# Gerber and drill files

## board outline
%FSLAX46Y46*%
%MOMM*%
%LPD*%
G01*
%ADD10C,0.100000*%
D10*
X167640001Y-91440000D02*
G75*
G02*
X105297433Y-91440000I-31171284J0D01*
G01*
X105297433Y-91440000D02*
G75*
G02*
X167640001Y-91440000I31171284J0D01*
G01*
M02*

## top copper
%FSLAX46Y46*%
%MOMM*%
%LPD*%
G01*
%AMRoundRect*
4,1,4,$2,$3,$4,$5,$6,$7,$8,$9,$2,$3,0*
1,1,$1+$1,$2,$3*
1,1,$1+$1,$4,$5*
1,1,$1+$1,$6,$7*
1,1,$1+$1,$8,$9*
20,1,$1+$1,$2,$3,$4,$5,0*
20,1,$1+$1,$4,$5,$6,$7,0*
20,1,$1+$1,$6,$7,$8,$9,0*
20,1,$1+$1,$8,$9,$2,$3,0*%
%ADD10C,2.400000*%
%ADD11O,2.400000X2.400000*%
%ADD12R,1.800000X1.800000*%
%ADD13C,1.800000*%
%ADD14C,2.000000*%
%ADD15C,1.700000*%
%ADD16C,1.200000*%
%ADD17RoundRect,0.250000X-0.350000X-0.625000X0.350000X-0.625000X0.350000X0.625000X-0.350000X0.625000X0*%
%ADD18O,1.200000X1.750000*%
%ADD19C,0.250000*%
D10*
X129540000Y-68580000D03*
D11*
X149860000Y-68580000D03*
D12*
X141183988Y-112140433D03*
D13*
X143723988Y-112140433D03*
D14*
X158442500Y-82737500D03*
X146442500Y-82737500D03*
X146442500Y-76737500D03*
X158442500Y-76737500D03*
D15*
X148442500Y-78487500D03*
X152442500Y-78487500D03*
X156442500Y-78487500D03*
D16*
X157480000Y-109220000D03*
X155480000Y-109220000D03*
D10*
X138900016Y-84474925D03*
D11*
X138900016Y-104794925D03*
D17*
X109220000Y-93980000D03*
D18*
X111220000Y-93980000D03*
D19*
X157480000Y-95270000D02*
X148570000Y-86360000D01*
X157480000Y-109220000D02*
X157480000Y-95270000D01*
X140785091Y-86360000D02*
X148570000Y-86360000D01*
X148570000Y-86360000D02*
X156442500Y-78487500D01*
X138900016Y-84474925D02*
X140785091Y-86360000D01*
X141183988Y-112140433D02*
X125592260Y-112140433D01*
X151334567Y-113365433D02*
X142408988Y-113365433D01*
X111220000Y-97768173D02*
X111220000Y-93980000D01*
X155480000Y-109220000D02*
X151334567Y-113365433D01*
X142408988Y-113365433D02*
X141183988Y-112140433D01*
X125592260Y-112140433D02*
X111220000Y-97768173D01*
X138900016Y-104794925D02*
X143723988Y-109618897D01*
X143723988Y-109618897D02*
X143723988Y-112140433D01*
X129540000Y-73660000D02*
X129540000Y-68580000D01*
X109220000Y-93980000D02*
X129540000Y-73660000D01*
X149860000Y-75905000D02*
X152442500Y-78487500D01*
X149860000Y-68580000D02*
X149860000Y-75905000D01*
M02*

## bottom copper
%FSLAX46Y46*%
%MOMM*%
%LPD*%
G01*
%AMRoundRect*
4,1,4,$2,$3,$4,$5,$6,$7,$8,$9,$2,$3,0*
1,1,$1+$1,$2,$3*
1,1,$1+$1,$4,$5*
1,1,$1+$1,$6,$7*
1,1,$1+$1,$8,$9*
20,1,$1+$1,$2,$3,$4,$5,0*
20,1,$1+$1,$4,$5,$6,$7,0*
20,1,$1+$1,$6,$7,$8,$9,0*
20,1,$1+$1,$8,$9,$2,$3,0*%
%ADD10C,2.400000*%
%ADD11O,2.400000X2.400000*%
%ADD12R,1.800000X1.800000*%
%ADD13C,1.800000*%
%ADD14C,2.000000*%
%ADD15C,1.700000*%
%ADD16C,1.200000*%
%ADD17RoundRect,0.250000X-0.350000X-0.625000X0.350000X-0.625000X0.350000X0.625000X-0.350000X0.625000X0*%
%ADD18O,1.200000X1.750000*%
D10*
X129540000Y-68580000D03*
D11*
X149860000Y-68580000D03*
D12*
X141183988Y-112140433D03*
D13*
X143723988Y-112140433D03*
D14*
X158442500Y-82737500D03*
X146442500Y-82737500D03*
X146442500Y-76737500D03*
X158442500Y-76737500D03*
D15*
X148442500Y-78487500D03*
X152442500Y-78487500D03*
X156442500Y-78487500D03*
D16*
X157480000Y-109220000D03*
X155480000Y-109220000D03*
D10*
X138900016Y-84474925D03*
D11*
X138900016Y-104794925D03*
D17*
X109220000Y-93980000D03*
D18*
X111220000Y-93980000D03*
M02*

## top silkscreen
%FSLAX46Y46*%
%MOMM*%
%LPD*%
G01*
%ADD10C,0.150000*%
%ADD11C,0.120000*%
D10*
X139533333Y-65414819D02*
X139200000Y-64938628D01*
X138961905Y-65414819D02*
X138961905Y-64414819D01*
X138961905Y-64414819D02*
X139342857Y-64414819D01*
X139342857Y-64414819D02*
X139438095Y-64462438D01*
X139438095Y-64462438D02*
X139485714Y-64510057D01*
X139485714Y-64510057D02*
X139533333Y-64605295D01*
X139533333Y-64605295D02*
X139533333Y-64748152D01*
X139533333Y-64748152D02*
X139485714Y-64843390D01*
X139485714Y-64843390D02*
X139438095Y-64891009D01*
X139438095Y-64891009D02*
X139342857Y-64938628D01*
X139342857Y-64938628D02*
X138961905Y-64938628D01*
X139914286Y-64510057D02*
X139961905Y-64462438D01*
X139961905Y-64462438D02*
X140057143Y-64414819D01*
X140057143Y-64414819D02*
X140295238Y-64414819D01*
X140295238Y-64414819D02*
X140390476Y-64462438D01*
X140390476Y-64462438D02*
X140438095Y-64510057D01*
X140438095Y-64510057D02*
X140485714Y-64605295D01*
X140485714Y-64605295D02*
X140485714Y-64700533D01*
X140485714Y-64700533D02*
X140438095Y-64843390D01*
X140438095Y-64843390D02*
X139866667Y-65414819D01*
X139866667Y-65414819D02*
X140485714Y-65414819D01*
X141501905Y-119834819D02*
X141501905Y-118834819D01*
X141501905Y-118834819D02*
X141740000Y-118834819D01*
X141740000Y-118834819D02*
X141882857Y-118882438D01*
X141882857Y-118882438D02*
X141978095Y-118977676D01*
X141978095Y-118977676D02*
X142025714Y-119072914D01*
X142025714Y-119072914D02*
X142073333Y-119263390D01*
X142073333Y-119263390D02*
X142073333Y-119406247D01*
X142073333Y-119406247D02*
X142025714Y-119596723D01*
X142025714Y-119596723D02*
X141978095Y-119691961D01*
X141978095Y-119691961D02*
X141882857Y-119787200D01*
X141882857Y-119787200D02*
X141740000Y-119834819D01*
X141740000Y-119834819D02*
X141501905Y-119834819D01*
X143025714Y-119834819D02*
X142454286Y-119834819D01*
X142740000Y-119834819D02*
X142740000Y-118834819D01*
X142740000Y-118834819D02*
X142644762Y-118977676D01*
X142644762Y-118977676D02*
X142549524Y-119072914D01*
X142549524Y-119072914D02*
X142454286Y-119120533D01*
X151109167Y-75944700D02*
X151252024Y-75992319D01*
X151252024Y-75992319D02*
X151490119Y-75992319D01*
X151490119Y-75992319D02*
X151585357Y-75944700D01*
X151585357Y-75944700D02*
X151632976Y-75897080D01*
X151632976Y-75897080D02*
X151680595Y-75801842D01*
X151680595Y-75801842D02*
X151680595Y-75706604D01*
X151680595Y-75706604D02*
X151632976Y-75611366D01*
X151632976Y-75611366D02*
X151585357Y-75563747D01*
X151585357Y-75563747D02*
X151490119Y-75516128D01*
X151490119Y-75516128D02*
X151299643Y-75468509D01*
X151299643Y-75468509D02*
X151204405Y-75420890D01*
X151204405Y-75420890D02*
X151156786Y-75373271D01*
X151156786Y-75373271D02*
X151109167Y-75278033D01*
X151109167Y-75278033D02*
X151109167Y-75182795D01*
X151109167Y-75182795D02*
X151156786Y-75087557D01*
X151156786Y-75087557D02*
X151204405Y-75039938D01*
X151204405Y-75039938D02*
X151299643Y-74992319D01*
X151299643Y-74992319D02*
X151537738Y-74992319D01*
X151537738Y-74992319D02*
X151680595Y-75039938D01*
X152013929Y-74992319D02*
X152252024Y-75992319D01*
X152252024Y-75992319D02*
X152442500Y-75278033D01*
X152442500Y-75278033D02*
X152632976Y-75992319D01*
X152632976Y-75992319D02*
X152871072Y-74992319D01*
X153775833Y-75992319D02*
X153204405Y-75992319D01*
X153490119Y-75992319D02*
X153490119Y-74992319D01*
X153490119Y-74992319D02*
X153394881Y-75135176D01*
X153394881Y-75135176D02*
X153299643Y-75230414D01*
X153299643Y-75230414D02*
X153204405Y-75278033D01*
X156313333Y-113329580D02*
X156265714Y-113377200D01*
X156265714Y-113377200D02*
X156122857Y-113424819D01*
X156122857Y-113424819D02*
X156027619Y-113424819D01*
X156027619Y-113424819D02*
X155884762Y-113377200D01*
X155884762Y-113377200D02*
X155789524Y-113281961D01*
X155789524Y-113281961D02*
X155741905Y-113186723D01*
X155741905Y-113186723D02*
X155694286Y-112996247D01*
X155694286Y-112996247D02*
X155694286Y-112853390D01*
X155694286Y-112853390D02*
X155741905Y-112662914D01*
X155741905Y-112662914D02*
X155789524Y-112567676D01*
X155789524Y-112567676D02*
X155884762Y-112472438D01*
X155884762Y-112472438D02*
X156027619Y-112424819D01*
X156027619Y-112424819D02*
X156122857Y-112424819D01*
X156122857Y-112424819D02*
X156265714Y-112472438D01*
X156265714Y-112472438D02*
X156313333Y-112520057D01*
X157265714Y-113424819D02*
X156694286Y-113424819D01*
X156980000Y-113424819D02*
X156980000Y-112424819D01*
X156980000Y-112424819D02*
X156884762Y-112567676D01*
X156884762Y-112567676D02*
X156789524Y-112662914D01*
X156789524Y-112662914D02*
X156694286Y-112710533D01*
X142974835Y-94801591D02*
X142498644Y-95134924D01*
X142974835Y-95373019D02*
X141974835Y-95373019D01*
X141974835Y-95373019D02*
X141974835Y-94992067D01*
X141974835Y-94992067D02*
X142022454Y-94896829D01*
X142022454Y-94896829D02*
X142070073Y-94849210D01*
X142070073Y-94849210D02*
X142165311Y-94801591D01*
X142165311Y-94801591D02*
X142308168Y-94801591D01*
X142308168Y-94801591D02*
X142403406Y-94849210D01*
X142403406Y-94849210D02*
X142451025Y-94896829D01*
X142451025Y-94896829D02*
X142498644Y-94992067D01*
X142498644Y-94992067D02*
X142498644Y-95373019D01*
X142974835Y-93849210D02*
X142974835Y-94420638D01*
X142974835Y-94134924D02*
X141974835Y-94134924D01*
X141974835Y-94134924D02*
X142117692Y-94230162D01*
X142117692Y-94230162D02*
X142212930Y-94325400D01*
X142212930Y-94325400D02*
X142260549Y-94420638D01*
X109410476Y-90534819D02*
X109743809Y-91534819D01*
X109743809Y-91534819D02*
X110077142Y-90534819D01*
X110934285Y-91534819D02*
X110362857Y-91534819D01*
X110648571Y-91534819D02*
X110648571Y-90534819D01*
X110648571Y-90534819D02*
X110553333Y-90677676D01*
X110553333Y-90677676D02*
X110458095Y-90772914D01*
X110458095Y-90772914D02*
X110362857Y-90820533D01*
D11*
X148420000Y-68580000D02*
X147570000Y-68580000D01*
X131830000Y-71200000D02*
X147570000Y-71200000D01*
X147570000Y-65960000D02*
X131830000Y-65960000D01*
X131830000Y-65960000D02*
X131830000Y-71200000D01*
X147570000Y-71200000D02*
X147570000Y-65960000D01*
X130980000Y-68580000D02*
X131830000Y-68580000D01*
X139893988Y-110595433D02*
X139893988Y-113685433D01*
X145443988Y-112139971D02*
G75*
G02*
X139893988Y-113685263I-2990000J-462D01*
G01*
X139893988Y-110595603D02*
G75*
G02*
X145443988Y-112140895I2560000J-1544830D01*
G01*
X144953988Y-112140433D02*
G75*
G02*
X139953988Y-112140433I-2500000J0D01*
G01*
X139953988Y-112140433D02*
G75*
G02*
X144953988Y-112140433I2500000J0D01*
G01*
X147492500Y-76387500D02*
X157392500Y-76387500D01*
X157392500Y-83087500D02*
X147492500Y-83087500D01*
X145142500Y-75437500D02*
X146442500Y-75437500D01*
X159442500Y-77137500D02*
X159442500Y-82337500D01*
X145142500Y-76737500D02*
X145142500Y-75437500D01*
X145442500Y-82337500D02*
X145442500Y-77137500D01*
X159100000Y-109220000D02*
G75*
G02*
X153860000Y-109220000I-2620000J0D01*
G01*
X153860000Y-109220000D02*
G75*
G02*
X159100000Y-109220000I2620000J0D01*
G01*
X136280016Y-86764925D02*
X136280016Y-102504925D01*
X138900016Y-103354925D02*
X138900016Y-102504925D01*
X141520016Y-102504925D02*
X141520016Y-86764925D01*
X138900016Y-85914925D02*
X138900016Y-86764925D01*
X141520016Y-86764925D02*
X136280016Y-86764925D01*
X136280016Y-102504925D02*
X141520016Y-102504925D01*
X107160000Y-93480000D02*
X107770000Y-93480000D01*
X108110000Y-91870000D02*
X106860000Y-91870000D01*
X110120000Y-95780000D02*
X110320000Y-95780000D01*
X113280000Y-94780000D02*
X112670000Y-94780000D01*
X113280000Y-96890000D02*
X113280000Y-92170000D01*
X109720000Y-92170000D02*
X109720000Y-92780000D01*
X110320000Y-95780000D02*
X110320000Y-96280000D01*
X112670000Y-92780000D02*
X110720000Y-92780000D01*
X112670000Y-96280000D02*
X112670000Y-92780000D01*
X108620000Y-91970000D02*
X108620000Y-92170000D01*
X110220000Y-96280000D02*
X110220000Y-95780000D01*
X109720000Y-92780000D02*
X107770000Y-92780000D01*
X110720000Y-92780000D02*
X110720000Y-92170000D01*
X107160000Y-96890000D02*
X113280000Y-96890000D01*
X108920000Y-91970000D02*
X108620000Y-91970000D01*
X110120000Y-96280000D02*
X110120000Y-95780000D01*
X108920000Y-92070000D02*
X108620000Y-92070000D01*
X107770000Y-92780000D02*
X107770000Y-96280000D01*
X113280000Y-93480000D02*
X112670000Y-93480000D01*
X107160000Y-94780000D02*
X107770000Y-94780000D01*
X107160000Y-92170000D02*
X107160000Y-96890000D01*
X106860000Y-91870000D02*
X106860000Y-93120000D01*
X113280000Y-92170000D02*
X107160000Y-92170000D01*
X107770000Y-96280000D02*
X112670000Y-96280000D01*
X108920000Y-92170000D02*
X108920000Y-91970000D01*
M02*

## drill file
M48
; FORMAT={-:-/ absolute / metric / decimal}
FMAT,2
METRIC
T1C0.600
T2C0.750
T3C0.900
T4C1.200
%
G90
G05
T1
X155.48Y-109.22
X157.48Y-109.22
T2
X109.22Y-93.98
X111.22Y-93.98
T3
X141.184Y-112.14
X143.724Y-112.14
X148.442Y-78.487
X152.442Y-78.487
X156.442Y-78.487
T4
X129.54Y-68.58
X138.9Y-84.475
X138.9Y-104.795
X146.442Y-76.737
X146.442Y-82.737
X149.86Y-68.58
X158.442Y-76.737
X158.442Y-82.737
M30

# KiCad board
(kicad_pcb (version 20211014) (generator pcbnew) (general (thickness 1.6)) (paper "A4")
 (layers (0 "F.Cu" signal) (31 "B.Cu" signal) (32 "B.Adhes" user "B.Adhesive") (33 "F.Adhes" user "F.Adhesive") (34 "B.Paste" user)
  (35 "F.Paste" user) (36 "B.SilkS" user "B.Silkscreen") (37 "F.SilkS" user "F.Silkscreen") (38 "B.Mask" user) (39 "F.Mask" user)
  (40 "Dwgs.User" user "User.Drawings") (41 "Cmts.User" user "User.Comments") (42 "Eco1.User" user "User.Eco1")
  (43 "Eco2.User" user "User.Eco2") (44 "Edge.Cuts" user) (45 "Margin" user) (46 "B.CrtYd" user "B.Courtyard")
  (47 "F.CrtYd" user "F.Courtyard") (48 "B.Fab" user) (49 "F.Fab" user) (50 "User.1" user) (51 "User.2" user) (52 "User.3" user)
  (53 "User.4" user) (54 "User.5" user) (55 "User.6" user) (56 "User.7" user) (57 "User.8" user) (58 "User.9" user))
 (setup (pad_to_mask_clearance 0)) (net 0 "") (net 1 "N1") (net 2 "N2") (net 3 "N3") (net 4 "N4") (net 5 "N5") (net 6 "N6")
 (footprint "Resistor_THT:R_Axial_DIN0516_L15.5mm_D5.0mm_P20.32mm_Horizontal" (layer "F.Cu") (at 129.54 68.58)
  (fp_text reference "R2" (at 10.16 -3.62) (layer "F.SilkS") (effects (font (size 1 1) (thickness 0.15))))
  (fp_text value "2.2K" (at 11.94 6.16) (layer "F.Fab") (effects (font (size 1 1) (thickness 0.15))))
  (fp_line (start 18.88 0) (end 18.03 0) (layer "F.SilkS") (width 0.12))
  (fp_line (start 2.29 2.62) (end 18.03 2.62) (layer "F.SilkS") (width 0.12))
  (fp_line (start 18.03 -2.62) (end 2.29 -2.62) (layer "F.SilkS") (width 0.12))
  (fp_line (start 2.29 -2.62) (end 2.29 2.62) (layer "F.SilkS") (width 0.12))
  (fp_line (start 18.03 2.62) (end 18.03 -2.62) (layer "F.SilkS") (width 0.12))
  (fp_line (start 1.44 0) (end 2.29 0) (layer "F.SilkS") (width 0.12))
  (pad "1" thru_hole circle (at 0 0) (size 2.4 2.4) (drill 1.2) (layers *.Cu *.Mask) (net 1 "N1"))
  (pad "2" thru_hole oval (at 20.32 0) (size 2.4 2.4) (drill 1.2) (layers *.Cu *.Mask) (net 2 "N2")))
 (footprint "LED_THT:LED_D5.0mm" (layer "F.Cu") (at 141.183988 112.140433)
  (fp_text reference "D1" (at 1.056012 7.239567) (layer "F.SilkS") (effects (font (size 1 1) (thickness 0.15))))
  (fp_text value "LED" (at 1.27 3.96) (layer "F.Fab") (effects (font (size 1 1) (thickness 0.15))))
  (fp_line (start -1.29 -1.545) (end -1.29 1.545) (layer "F.SilkS") (width 0.12))
  (fp_arc (start 4.26 -0.000462) (mid 2.072002 2.880433) (end -1.29 1.54483) (layer "F.SilkS") (width 0.12))
  (fp_arc (start -1.29 -1.54483) (mid 2.072002 -2.880433) (end 4.26 0.000462) (layer "F.SilkS") (width 0.12))
  (fp_circle (center 1.27 0) (end 3.77 0) (layer "F.SilkS") (width 0.12) (fill none))
  (pad "1" thru_hole rect (at 0 0) (size 1.8 1.8) (drill 0.9) (layers *.Cu *.Mask) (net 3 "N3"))
  (pad "2" thru_hole circle (at 2.54 0) (size 1.8 1.8) (drill 0.9) (layers *.Cu *.Mask) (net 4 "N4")))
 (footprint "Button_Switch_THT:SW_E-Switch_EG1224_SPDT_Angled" (layer "F.Cu") (at 148.4425 78.4875)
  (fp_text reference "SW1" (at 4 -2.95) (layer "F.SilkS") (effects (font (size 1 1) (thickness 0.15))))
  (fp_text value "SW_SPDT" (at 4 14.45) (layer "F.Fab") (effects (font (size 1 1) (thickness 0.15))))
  (fp_line (start -0.95 -2.1) (end 8.95 -2.1) (layer "F.SilkS") (width 0.12))
  (fp_line (start 8.95 4.6) (end -0.95 4.6) (layer "F.SilkS") (width 0.12))
  (fp_line (start -3.3 -3.05) (end -2 -3.05) (layer "F.SilkS") (width 0.12))
  (fp_line (start 11 -1.35) (end 11 3.85) (layer "F.SilkS") (width 0.12))
  (fp_line (start -3.3 -1.75) (end -3.3 -3.05) (layer "F.SilkS") (width 0.12))
  (fp_line (start -3 3.85) (end -3 -1.35) (layer "F.SilkS") (width 0.12))
  (pad "" thru_hole circle (at 10 4.25) (size 2 2) (drill 1.2) (layers *.Cu *.Mask))
  (pad "" thru_hole circle (at -2 4.25) (size 2 2) (drill 1.2) (layers *.Cu *.Mask))
  (pad "" thru_hole circle (at -2 -1.75) (size 2 2) (drill 1.2) (layers *.Cu *.Mask))
  (pad "" thru_hole circle (at 10 -1.75) (size 2 2) (drill 1.2) (layers *.Cu *.Mask))
  (pad "1" thru_hole circle (at 0 0) (size 1.7 1.7) (drill 0.9) (layers *.Cu *.Mask) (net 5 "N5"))
  (pad "2" thru_hole circle (at 4 0) (size 1.7 1.7) (drill 0.9) (layers *.Cu *.Mask) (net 2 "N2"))
  (pad "3" thru_hole circle (at 8 0) (size 1.7 1.7) (drill 0.9) (layers *.Cu *.Mask) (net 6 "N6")))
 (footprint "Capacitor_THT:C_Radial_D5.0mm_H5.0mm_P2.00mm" (layer "F.Cu") (at 157.48 109.22 180)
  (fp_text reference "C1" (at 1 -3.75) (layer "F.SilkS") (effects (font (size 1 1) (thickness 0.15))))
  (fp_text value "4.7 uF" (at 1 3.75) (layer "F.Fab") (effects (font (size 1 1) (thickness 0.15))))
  (fp_circle (center 1 0) (end 3.62 0) (layer "F.SilkS") (width 0.12) (fill none))
  (pad "1" thru_hole circle (at 0 0 180) (size 1.2 1.2) (drill 0.6) (layers *.Cu *.Mask) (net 6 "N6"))
  (pad "2" thru_hole circle (at 2 0 180) (size 1.2 1.2) (drill 0.6) (layers *.Cu *.Mask) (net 3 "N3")))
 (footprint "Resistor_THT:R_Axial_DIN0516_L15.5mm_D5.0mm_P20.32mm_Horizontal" (layer "F.Cu") (at 138.900016 84.474925 -90)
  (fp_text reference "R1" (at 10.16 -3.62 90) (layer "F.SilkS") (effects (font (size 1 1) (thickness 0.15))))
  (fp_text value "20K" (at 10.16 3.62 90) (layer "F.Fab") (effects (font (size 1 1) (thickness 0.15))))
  (fp_line (start 2.29 2.62) (end 18.03 2.62) (layer "F.SilkS") (width 0.12))
  (fp_line (start 18.88 0) (end 18.03 0) (layer "F.SilkS") (width 0.12))
  (fp_line (start 18.03 -2.62) (end 2.29 -2.62) (layer "F.SilkS") (width 0.12))
  (fp_line (start 1.44 0) (end 2.29 0) (layer "F.SilkS") (width 0.12))
  (fp_line (start 2.29 -2.62) (end 2.29 2.62) (layer "F.SilkS") (width 0.12))
  (fp_line (start 18.03 2.62) (end 18.03 -2.62) (layer "F.SilkS") (width 0.12))
  (pad "1" thru_hole circle (at 0 0 270) (size 2.4 2.4) (drill 1.2) (layers *.Cu *.Mask) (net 6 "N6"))
  (pad "2" thru_hole oval (at 20.32 0 270) (size 2.4 2.4) (drill 1.2) (layers *.Cu *.Mask) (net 4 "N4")))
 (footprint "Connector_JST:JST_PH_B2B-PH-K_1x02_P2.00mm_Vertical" (layer "F.Cu") (at 109.22 93.98)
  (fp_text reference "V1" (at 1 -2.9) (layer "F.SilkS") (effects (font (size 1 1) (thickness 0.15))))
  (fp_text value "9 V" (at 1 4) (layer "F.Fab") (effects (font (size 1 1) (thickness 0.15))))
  (fp_line (start -2.06 -0.5) (end -1.45 -0.5) (layer "F.SilkS") (width 0.12))
  (fp_line (start -1.11 -2.11) (end -2.36 -2.11) (layer "F.SilkS") (width 0.12))
  (fp_line (start 0.9 1.8) (end 1.1 1.8) (layer "F.SilkS") (width 0.12))
  (fp_line (start 4.06 0.8) (end 3.45 0.8) (layer "F.SilkS") (width 0.12))
  (fp_line (start 4.06 2.91) (end 4.06 -1.81) (layer "F.SilkS") (width 0.12))
  (fp_line (start 0.5 -1.81) (end 0.5 -1.2) (layer "F.SilkS") (width 0.12))
  (fp_line (start 1.1 1.8) (end 1.1 2.3) (layer "F.SilkS") (width 0.12))
  (fp_line (start 3.45 -1.2) (end 1.5 -1.2) (layer "F.SilkS") (width 0.12))
  (fp_line (start 3.45 2.3) (end 3.45 -1.2) (layer "F.SilkS") (width 0.12))
  (fp_line (start -0.6 -2.01) (end -0.6 -1.81) (layer "F.SilkS") (width 0.12))
  (fp_line (start 1 2.3) (end 1 1.8) (layer "F.SilkS") (width 0.12))
  (fp_line (start 0.5 -1.2) (end -1.45 -1.2) (layer "F.SilkS") (width 0.12))
  (fp_line (start 1.5 -1.2) (end 1.5 -1.81) (layer "F.SilkS") (width 0.12))
  (fp_line (start -2.06 2.91) (end 4.06 2.91) (layer "F.SilkS") (width 0.12))
  (fp_line (start -0.3 -2.01) (end -0.6 -2.01) (layer "F.SilkS") (width 0.12))
  (fp_line (start 0.9 2.3) (end 0.9 1.8) (layer "F.SilkS") (width 0.12))
  (fp_line (start -0.3 -1.91) (end -0.6 -1.91) (layer "F.SilkS") (width 0.12))
  (fp_line (start -1.45 -1.2) (end -1.45 2.3) (layer "F.SilkS") (width 0.12))
  (fp_line (start 4.06 -0.5) (end 3.45 -0.5) (layer "F.SilkS") (width 0.12))
  (fp_line (start -2.06 0.8) (end -1.45 0.8) (layer "F.SilkS") (width 0.12))
  (fp_line (start -2.06 -1.81) (end -2.06 2.91) (layer "F.SilkS") (width 0.12))
  (fp_line (start -2.36 -2.11) (end -2.36 -0.86) (layer "F.SilkS") (width 0.12))
  (fp_line (start 4.06 -1.81) (end -2.06 -1.81) (layer "F.SilkS") (width 0.12))
  (fp_line (start -1.45 2.3) (end 3.45 2.3) (layer "F.SilkS") (width 0.12))
  (fp_line (start -0.3 -1.81) (end -0.3 -2.01) (layer "F.SilkS") (width 0.12))
  (pad "1" thru_hole roundrect (at 0 0) (size 1.2 1.75) (drill 0.75) (layers *.Cu *.Mask) (roundrect_rratio 0.208333) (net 1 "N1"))
  (pad "2" thru_hole oval (at 2 0) (size 1.2 1.75) (drill 0.75) (layers *.Cu *.Mask) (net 3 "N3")))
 (gr_circle (center 136.468717 91.44) (end 163.660468 106.68) (layer "Edge.Cuts") (width 0.1) (fill none))
 (segment (start 157.48 95.27) (end 148.57 86.36) (width 0.25) (layer "F.Cu") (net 6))
 (segment (start 157.48 109.22) (end 157.48 95.27) (width 0.25) (layer "F.Cu") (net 6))
 (segment (start 140.785091 86.36) (end 148.57 86.36) (width 0.25) (layer "F.Cu") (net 6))
 (segment (start 148.57 86.36) (end 156.4425 78.4875) (width 0.25) (layer "F.Cu") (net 6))
 (segment (start 138.900016 84.474925) (end 140.785091 86.36) (width 0.25) (layer "F.Cu") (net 6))
 (segment (start 141.183988 112.140433) (end 125.59226 112.140433) (width 0.25) (layer "F.Cu") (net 3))
 (segment (start 151.334567 113.365433) (end 142.408988 113.365433) (width 0.25) (layer "F.Cu") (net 3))
 (segment (start 111.22 97.768173) (end 111.22 93.98) (width 0.25) (layer "F.Cu") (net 3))
 (segment (start 155.48 109.22) (end 151.334567 113.365433) (width 0.25) (layer "F.Cu") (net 3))
 (segment (start 142.408988 113.365433) (end 141.183988 112.140433) (width 0.25) (layer "F.Cu") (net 3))
 (segment (start 125.59226 112.140433) (end 111.22 97.768173) (width 0.25) (layer "F.Cu") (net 3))
 (segment (start 138.900016 104.794925) (end 143.723988 109.618897) (width 0.25) (layer "F.Cu") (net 4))
 (segment (start 143.723988 109.618897) (end 143.723988 112.140433) (width 0.25) (layer "F.Cu") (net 4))
 (segment (start 129.54 73.66) (end 129.54 68.58) (width 0.25) (layer "F.Cu") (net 1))
 (segment (start 109.22 93.98) (end 129.54 73.66) (width 0.25) (layer "F.Cu") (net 1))
 (segment (start 149.86 75.905) (end 152.4425 78.4875) (width 0.25) (layer "F.Cu") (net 2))
 (segment (start 149.86 68.58) (end 149.86 75.905) (width 0.25) (layer "F.Cu") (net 2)))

